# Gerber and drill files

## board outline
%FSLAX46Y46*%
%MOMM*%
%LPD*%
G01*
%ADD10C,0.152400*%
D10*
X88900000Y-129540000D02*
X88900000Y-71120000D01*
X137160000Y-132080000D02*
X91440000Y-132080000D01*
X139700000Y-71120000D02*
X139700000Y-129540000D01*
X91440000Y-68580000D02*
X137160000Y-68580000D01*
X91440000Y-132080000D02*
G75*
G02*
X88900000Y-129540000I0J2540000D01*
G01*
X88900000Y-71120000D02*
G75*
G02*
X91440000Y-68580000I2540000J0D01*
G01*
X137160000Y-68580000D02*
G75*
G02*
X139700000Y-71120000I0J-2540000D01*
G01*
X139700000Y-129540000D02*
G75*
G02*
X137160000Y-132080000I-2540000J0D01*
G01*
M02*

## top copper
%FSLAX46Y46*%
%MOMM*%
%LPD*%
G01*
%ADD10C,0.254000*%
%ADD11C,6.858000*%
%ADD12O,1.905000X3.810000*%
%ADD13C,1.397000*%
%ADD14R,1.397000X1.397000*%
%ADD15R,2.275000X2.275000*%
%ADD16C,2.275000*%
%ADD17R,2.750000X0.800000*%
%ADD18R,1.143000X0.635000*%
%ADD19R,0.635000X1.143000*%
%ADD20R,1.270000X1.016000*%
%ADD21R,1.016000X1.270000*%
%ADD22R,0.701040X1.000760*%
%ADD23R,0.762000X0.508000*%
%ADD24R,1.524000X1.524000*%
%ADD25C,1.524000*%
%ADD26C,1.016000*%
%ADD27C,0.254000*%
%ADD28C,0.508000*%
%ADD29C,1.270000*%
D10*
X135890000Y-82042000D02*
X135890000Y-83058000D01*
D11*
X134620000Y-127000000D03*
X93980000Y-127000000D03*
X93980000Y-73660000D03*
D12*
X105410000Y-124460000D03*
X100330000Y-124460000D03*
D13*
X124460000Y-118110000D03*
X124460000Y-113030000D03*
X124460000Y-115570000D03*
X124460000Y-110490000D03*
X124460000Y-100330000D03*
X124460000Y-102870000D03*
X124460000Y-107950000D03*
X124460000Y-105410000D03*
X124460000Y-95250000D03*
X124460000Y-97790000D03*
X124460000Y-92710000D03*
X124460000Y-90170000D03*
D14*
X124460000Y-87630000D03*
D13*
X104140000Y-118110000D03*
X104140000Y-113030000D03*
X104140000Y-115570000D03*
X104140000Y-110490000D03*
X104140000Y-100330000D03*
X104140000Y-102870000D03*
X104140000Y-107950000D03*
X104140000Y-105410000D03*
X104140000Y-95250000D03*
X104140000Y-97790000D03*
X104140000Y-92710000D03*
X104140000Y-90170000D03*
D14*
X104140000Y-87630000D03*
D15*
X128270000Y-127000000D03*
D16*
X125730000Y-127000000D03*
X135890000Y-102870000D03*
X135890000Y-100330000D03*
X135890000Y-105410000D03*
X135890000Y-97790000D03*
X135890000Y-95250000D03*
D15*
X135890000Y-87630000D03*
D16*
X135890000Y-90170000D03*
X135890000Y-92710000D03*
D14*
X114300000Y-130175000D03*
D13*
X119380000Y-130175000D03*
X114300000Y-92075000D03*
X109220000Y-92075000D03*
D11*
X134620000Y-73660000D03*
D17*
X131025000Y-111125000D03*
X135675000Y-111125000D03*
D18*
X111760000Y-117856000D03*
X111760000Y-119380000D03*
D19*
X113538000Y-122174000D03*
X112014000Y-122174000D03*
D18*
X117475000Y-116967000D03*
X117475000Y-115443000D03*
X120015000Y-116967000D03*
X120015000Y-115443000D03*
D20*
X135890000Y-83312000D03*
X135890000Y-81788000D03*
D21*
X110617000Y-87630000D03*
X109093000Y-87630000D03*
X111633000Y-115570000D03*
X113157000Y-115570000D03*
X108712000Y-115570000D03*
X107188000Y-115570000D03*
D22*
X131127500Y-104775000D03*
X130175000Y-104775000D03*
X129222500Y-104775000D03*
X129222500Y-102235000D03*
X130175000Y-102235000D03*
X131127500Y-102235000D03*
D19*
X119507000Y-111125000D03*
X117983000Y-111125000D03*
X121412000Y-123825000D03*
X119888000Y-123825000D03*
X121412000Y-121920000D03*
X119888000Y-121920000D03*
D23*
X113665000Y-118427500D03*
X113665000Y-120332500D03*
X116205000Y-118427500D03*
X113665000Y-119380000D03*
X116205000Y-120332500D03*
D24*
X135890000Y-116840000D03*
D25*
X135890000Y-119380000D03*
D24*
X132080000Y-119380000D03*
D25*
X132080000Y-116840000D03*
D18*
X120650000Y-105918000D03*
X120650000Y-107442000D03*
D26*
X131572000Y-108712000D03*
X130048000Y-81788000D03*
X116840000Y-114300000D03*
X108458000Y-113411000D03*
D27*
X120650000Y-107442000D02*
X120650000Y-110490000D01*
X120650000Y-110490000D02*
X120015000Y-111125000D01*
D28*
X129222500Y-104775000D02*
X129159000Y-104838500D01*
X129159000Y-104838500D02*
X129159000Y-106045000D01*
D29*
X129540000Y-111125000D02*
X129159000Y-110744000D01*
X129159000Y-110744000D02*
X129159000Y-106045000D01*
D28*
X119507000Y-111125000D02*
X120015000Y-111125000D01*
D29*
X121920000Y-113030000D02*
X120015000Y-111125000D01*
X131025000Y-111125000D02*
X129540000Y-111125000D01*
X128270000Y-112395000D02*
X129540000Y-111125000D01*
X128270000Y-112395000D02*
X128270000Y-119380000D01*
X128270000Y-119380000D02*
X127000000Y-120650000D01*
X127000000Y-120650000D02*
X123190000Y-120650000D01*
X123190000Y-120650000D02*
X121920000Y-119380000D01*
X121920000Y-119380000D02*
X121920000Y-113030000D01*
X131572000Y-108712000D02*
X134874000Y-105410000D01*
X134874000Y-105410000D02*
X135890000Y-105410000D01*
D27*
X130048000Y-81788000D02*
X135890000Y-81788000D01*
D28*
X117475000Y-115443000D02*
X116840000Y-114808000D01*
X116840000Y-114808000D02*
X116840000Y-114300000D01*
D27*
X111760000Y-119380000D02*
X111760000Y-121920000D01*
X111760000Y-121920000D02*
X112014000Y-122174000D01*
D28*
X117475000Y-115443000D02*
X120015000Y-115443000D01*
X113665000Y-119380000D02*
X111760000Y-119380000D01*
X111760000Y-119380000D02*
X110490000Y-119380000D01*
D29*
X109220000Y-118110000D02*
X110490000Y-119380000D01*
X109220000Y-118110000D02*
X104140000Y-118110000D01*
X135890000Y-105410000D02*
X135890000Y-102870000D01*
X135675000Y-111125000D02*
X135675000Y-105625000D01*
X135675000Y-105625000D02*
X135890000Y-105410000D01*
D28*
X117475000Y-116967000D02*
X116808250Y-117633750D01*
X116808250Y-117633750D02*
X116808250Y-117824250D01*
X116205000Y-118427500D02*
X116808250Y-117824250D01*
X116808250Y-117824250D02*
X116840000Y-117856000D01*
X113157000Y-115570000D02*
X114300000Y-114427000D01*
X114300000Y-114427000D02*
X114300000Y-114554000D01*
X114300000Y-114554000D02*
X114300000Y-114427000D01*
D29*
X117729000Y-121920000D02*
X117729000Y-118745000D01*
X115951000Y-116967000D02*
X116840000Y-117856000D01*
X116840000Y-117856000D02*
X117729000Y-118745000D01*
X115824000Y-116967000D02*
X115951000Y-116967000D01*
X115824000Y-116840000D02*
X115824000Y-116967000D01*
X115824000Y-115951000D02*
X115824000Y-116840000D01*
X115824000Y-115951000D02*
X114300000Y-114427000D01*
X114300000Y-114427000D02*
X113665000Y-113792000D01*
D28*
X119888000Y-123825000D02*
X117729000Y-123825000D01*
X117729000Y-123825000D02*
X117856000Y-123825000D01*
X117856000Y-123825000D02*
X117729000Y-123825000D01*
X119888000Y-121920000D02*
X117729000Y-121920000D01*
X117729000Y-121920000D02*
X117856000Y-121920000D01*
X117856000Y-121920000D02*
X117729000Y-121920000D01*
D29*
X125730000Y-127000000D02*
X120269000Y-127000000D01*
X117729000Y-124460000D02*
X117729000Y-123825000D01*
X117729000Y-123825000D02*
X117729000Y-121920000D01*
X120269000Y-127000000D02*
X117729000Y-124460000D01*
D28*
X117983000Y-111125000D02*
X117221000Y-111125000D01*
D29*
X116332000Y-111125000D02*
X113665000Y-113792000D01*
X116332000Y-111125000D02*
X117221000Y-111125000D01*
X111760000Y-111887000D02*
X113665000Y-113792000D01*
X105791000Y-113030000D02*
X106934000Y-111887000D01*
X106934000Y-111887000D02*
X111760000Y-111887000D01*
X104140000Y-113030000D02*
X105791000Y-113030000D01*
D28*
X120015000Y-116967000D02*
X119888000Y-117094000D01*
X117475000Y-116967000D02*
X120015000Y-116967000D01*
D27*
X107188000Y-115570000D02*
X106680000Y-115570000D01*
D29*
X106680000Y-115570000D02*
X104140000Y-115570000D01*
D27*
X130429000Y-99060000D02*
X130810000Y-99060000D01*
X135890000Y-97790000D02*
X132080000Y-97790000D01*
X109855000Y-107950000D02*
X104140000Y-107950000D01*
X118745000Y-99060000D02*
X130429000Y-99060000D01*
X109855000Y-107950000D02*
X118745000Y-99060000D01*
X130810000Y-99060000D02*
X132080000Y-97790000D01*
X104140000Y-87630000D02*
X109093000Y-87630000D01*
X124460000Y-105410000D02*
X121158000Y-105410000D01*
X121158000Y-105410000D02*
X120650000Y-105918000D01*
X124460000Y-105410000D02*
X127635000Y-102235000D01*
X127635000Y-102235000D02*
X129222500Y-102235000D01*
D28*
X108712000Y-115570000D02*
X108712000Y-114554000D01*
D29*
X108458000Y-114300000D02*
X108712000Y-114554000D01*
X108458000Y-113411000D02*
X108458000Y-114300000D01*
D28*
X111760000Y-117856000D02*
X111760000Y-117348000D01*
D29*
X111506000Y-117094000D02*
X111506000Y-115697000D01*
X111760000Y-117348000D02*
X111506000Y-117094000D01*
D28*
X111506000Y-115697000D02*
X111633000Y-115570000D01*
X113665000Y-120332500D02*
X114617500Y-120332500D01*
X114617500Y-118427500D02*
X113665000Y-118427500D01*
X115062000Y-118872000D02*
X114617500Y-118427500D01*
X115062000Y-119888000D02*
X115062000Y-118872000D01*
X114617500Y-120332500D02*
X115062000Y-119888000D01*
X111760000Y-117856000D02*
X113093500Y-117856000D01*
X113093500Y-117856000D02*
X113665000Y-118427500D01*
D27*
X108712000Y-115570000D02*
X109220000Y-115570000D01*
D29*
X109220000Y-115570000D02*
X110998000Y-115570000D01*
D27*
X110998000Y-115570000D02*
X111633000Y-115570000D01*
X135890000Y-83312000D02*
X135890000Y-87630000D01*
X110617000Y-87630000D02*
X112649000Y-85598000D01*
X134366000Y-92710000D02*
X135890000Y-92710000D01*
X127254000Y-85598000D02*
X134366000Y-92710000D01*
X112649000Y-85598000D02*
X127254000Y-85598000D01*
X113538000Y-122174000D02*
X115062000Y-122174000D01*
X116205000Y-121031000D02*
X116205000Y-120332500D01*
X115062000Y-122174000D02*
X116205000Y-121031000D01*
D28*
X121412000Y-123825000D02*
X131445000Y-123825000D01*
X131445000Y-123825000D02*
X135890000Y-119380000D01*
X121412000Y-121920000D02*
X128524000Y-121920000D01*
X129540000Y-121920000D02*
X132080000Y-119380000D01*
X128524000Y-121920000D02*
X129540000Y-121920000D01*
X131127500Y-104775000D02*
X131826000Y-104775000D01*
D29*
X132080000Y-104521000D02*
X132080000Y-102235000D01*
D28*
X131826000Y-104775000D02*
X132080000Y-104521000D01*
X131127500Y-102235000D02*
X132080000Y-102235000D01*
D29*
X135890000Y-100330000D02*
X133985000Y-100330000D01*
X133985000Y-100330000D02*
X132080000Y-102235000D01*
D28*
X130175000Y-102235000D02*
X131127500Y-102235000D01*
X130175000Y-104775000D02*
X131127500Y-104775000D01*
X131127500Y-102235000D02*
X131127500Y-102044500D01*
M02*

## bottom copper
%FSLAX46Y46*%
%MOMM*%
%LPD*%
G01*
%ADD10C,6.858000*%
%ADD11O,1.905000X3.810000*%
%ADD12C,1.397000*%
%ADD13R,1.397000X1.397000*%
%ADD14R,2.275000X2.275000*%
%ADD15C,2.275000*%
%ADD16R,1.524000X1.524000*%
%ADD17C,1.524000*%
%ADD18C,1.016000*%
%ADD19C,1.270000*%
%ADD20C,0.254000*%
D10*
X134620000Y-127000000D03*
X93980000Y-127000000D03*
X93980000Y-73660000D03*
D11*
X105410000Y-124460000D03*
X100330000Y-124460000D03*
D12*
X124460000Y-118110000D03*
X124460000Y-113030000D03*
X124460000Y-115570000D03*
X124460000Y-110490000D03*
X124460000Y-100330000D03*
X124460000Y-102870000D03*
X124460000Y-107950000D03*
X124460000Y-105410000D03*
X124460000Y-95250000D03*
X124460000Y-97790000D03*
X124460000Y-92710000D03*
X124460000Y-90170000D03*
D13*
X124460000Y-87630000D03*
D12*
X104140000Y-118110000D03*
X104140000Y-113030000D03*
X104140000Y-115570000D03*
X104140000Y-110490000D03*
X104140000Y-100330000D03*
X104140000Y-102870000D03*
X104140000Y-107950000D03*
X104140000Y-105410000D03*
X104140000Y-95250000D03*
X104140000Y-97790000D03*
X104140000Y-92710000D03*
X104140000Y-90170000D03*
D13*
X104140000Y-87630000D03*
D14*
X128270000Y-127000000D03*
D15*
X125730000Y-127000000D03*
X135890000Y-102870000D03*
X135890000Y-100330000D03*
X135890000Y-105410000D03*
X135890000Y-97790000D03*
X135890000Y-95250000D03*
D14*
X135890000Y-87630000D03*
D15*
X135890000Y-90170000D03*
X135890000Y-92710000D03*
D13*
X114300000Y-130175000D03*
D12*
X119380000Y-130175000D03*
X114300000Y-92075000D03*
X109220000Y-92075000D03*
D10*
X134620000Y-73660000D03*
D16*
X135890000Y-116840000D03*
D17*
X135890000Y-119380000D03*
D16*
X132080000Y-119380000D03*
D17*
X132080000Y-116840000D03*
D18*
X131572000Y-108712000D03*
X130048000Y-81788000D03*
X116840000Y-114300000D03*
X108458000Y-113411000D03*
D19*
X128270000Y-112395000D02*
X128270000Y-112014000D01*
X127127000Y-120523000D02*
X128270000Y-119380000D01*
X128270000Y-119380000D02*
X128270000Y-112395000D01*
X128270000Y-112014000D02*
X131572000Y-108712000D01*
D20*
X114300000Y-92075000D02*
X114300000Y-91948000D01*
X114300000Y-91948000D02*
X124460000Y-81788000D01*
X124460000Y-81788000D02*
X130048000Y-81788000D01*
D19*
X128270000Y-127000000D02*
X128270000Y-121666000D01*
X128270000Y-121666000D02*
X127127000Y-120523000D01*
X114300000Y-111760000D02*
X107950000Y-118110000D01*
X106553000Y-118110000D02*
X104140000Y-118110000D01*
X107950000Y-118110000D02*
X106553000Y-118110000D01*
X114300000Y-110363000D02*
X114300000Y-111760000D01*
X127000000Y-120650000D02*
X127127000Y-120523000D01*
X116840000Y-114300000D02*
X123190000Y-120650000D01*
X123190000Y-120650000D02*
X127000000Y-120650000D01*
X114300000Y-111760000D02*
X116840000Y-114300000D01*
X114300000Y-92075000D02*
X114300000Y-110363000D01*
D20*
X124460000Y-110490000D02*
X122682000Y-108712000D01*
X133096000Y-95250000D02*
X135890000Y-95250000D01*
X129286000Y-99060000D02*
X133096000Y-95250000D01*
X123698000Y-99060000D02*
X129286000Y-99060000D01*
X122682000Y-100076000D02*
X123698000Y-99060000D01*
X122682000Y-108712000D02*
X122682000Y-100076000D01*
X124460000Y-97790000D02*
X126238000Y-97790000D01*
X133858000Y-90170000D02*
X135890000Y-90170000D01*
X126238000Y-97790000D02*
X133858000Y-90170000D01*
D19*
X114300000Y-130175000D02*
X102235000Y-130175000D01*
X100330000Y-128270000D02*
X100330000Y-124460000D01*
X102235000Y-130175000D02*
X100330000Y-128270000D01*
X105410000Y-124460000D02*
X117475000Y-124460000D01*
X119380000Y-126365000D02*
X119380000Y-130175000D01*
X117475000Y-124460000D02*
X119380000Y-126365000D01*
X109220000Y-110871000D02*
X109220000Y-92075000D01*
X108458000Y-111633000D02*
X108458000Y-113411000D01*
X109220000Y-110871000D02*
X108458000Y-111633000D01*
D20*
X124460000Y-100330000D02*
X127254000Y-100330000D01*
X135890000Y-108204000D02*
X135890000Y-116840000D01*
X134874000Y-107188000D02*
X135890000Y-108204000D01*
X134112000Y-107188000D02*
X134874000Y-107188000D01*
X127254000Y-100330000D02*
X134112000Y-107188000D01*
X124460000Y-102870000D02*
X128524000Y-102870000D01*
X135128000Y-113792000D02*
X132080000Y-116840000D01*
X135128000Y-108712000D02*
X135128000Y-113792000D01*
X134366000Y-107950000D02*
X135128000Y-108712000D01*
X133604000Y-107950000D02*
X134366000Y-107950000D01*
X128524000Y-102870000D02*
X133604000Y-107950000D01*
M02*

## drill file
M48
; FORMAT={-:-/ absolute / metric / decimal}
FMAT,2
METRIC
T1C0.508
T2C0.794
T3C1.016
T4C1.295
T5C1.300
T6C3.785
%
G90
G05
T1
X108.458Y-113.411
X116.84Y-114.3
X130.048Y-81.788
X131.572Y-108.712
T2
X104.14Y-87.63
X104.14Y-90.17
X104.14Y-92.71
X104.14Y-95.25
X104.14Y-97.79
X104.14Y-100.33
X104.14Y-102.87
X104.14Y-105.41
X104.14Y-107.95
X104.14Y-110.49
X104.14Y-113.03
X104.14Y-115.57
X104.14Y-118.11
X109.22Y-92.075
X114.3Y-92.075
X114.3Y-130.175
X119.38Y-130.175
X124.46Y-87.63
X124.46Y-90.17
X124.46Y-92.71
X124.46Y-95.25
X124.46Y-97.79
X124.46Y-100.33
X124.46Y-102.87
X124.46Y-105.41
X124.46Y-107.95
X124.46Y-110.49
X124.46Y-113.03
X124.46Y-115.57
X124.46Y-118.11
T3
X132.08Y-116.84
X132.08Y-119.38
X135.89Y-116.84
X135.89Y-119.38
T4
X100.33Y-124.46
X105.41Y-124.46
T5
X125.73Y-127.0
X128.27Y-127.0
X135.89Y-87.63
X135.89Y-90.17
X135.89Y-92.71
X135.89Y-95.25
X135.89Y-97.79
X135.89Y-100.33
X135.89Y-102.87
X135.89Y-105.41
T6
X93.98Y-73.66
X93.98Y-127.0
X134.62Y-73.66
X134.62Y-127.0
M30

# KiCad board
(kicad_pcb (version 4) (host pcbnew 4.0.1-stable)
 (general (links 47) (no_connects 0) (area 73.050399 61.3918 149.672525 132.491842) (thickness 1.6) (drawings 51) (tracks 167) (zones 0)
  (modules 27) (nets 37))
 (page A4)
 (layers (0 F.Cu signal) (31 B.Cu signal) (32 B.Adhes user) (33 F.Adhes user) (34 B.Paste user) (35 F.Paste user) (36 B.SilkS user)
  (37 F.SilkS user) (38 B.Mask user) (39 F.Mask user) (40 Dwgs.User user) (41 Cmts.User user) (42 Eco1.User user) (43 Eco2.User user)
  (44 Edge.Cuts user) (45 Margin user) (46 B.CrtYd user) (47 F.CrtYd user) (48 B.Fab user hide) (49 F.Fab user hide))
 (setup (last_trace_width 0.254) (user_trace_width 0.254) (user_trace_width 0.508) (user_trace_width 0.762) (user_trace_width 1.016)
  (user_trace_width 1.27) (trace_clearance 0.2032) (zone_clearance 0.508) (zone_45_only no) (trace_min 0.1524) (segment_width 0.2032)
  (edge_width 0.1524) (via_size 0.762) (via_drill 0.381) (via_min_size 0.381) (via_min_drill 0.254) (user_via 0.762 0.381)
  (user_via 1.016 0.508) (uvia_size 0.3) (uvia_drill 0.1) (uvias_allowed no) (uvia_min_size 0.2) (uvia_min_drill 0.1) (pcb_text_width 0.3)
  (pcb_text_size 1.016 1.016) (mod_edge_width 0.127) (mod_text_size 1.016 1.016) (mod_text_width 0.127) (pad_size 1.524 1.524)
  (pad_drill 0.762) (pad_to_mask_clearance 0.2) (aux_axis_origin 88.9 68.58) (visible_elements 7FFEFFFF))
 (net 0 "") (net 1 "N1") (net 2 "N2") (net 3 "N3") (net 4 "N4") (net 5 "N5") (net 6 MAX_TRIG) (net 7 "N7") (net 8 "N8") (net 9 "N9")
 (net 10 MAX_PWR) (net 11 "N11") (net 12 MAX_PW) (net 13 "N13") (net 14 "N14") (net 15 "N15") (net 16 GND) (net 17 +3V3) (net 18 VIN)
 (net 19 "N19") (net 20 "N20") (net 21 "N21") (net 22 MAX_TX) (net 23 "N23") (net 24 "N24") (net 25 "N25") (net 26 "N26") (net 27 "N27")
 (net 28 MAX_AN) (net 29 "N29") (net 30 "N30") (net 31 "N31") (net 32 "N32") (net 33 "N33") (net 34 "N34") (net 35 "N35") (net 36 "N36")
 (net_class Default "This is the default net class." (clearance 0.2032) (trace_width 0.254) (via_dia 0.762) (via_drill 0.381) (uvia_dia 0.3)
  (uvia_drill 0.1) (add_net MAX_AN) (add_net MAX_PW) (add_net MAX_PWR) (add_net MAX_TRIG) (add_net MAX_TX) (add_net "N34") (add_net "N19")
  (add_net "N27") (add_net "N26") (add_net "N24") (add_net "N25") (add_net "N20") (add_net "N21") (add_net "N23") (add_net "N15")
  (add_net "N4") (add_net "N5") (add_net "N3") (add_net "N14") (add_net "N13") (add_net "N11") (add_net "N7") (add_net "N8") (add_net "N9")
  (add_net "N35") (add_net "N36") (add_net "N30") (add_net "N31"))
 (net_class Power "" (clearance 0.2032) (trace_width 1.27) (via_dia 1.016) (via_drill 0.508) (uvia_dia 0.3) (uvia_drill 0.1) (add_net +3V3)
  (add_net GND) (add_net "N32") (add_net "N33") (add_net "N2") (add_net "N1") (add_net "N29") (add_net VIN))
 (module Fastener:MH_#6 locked (layer F.Cu) (at 134.62 127)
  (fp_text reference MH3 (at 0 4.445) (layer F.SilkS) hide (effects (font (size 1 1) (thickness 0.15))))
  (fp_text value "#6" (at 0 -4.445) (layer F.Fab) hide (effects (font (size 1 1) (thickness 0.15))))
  (pad 1 thru_hole circle (at 0 0) (size 6.858 6.858) (drill 3.7846) (layers *.Cu *.Mask F.SilkS)))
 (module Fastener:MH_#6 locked (layer F.Cu) (at 93.98 127)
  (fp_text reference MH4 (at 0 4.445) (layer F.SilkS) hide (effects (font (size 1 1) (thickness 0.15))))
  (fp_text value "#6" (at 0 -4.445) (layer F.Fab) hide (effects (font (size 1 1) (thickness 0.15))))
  (pad 1 thru_hole circle (at 0 0) (size 6.858 6.858) (drill 3.7846) (layers *.Cu *.Mask F.SilkS)))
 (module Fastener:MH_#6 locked (layer F.Cu) (at 93.98 73.66)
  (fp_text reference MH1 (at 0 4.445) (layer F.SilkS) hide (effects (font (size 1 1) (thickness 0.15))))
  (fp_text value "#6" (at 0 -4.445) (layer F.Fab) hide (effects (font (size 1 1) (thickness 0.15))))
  (pad 1 thru_hole circle (at 0 0) (size 6.858 6.858) (drill 3.7846) (layers *.Cu *.Mask F.SilkS)))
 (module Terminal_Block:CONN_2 (layer F.Cu) (at 102.87 124.46 180)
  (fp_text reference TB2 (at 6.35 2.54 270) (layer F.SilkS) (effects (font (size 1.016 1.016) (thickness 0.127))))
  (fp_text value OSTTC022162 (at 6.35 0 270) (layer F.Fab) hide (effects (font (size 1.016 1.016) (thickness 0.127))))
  (pad 1 thru_hole oval (at -2.54 0 180) (size 1.905 3.81) (drill 1.2954) (layers *.Cu F.Paste F.SilkS F.Mask) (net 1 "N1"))
  (pad 2 thru_hole oval (at 2.54 0 180) (size 1.905 3.81) (drill 1.2954) (layers *.Cu F.Paste F.SilkS F.Mask) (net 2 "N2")))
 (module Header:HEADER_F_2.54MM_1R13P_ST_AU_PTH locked (layer F.Cu) (at 124.46 102.87 270)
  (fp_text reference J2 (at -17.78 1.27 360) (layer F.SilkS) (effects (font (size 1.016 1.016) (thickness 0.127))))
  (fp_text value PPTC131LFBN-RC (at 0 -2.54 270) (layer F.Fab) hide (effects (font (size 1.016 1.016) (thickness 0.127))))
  (pad 13 thru_hole circle (at 15.24 0 270) (size 1.397 1.397) (drill 0.79375) (layers *.Cu *.Mask F.SilkS) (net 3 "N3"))
  (pad 11 thru_hole circle (at 10.16 0 270) (size 1.397 1.397) (drill 0.79375) (layers *.Cu *.Mask F.SilkS) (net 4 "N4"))
  (pad 12 thru_hole circle (at 12.7 0 270) (size 1.397 1.397) (drill 0.79375) (layers *.Cu *.Mask F.SilkS) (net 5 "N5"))
  (pad 10 thru_hole circle (at 7.62 0 270) (size 1.397 1.397) (drill 0.79375) (layers *.Cu *.Mask F.SilkS) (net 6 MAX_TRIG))
  (pad 6 thru_hole circle (at -2.54 0 270) (size 1.397 1.397) (drill 0.79375) (layers *.Cu *.Mask F.SilkS) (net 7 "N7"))
  (pad 7 thru_hole circle (at 0 0 270) (size 1.397 1.397) (drill 0.79375) (layers *.Cu *.Mask F.SilkS) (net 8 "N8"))
  (pad 9 thru_hole circle (at 5.08 0 270) (size 1.397 1.397) (drill 0.79375) (layers *.Cu *.Mask F.SilkS) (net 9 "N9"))
  (pad 8 thru_hole circle (at 2.54 0 270) (size 1.397 1.397) (drill 0.79375) (layers *.Cu *.Mask F.SilkS) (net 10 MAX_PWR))
  (pad 4 thru_hole circle (at -7.62 0 270) (size 1.397 1.397) (drill 0.79375) (layers *.Cu *.Mask F.SilkS) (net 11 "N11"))
  (pad 5 thru_hole circle (at -5.08 0 270) (size 1.397 1.397) (drill 0.79375) (layers *.Cu *.Mask F.SilkS) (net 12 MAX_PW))
  (pad 3 thru_hole circle (at -10.16 0 270) (size 1.397 1.397) (drill 0.79375) (layers *.Cu *.Mask F.SilkS) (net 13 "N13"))
  (pad 2 thru_hole circle (at -12.7 0 270) (size 1.397 1.397) (drill 0.79375) (layers *.Cu *.Mask F.SilkS) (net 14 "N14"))
  (pad 1 thru_hole rect (at -15.24 0 270) (size 1.397 1.397) (drill 0.79375) (layers *.Cu *.Mask F.SilkS) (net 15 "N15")))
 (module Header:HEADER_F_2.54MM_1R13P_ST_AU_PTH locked (layer F.Cu) (at 104.14 102.87 270)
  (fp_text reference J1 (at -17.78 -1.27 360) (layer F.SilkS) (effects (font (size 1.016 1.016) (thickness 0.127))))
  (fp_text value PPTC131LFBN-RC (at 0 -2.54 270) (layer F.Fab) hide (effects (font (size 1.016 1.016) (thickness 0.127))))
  (pad 13 thru_hole circle (at 15.24 0 270) (size 1.397 1.397) (drill 0.79375) (layers *.Cu *.Mask F.SilkS) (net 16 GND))
  (pad 11 thru_hole circle (at 10.16 0 270) (size 1.397 1.397) (drill 0.79375) (layers *.Cu *.Mask F.SilkS) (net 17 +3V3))
  (pad 12 thru_hole circle (at 12.7 0 270) (size 1.397 1.397) (drill 0.79375) (layers *.Cu *.Mask F.SilkS) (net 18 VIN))
  (pad 10 thru_hole circle (at 7.62 0 270) (size 1.397 1.397) (drill 0.79375) (layers *.Cu *.Mask F.SilkS) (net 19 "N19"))
  (pad 6 thru_hole circle (at -2.54 0 270) (size 1.397 1.397) (drill 0.79375) (layers *.Cu *.Mask F.SilkS) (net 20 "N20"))
  (pad 7 thru_hole circle (at 0 0 270) (size 1.397 1.397) (drill 0.79375) (layers *.Cu *.Mask F.SilkS) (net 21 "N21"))
  (pad 9 thru_hole circle (at 5.08 0 270) (size 1.397 1.397) (drill 0.79375) (layers *.Cu *.Mask F.SilkS) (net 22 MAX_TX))
  (pad 8 thru_hole circle (at 2.54 0 270) (size 1.397 1.397) (drill 0.79375) (layers *.Cu *.Mask F.SilkS) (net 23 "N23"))
  (pad 4 thru_hole circle (at -7.62 0 270) (size 1.397 1.397) (drill 0.79375) (layers *.Cu *.Mask F.SilkS) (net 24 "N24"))
  (pad 5 thru_hole circle (at -5.08 0 270) (size 1.397 1.397) (drill 0.79375) (layers *.Cu *.Mask F.SilkS) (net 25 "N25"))
  (pad 3 thru_hole circle (at -10.16 0 270) (size 1.397 1.397) (drill 0.79375) (layers *.Cu *.Mask F.SilkS) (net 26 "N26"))
  (pad 2 thru_hole circle (at -12.7 0 270) (size 1.397 1.397) (drill 0.79375) (layers *.Cu *.Mask F.SilkS) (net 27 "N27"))
  (pad 1 thru_hole rect (at -15.24 0 270) (size 1.397 1.397) (drill 0.79375) (layers *.Cu *.Mask F.SilkS) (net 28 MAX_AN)))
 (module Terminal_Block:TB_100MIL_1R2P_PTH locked (layer F.Cu) (at 127 127 180)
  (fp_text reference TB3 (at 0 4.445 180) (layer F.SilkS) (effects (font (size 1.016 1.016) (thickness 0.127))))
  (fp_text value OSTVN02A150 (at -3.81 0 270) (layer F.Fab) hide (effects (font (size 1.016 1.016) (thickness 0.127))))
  (pad 1 thru_hole rect (at -1.27 0 180) (size 2.275 2.275) (drill 1.3) (layers *.Cu *.Mask F.SilkS) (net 16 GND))
  (pad 2 thru_hole circle (at 1.27 0 180) (size 2.275 2.275) (drill 1.3) (layers *.Cu *.Mask F.SilkS) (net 17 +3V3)))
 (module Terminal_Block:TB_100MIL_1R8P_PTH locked (layer F.Cu) (at 135.89 96.52 270)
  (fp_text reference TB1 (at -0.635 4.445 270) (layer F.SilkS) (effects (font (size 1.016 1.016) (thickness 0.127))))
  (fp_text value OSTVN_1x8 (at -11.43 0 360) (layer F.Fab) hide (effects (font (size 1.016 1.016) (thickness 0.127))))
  (pad 7 thru_hole circle (at 6.35 0 270) (size 2.275 2.275) (drill 1.3) (layers *.Cu *.Mask F.SilkS) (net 16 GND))
  (pad 6 thru_hole circle (at 3.81 0 270) (size 2.275 2.275) (drill 1.3) (layers *.Cu *.Mask F.SilkS) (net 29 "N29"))
  (pad 8 thru_hole circle (at 8.89 0 270) (size 2.275 2.275) (drill 1.3) (layers *.Cu *.Mask F.SilkS) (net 16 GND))
  (pad 5 thru_hole circle (at 1.27 0 270) (size 2.275 2.275) (drill 1.3) (layers *.Cu *.Mask F.SilkS) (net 22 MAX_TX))
  (pad 4 thru_hole circle (at -1.27 0 270) (size 2.275 2.275) (drill 1.3) (layers *.Cu *.Mask F.SilkS) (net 6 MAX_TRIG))
  (pad 1 thru_hole rect (at -8.89 0 270) (size 2.275 2.275) (drill 1.3) (layers *.Cu *.Mask F.SilkS) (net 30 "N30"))
  (pad 2 thru_hole circle (at -6.35 0 270) (size 2.275 2.275) (drill 1.3) (layers *.Cu *.Mask F.SilkS) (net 12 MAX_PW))
  (pad 3 thru_hole circle (at -3.81 0 270) (size 2.275 2.275) (drill 1.3) (layers *.Cu *.Mask F.SilkS) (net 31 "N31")))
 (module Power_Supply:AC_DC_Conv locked (layer B.Cu) (at 114.3 111.125 90)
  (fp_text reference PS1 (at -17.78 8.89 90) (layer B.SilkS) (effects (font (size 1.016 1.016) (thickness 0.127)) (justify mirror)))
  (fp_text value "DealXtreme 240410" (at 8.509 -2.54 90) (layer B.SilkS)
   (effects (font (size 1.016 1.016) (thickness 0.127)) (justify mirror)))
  (pad 1 thru_hole rect (at -19.05 0 90) (size 1.397 1.397) (drill 0.79375) (layers *.Cu *.Mask B.SilkS) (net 2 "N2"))
  (pad 2 thru_hole circle (at -19.05 5.08 90) (size 1.397 1.397) (drill 0.79375) (layers *.Cu *.Mask B.SilkS) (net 1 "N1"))
  (pad 4 thru_hole circle (at 19.05 0 90) (size 1.397 1.397) (drill 0.79375) (layers *.Cu *.Mask B.SilkS) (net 16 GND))
  (pad 3 thru_hole circle (at 19.05 -5.08 90) (size 1.397 1.397) (drill 0.79375) (layers *.Cu *.Mask B.SilkS) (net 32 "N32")))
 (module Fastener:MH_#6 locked (layer F.Cu) (at 134.62 73.66)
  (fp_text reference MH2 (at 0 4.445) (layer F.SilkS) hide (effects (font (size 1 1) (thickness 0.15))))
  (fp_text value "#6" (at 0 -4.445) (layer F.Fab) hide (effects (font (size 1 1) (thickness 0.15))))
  (pad 1 thru_hole circle (at 0 0) (size 6.858 6.858) (drill 3.7846) (layers *.Cu *.Mask F.SilkS)))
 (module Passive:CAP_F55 (layer F.Cu) (at 133.35 111.125 90)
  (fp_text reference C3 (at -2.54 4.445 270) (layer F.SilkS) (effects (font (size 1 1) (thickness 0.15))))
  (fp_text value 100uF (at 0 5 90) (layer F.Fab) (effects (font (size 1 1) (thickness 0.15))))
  (pad 1 smd rect (at 0 -2.325 90) (size 0.8 2.75) (layers F.Cu F.Paste F.Mask) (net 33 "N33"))
  (pad 2 smd rect (at 0 2.325 90) (size 0.8 2.75) (layers F.Cu F.Paste F.Mask) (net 16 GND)))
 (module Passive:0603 (layer F.Cu) (at 111.76 118.618 270)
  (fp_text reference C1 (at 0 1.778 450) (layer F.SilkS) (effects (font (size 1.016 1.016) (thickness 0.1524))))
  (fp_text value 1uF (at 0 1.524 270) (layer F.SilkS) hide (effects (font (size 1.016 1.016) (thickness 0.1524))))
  (pad 1 smd rect (at -0.762 0 270) (size 0.635 1.143) (layers F.Cu F.Paste F.Mask) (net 32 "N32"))
  (pad 2 smd rect (at 0.762 0 270) (size 0.635 1.143) (layers F.Cu F.Paste F.Mask) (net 16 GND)))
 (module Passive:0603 (layer F.Cu) (at 112.776 122.174 180)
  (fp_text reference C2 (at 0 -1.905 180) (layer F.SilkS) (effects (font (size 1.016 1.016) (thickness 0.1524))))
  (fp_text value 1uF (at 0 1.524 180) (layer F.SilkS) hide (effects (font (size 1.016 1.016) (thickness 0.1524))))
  (pad 1 smd rect (at -0.762 0 180) (size 0.635 1.143) (layers F.Cu F.Paste F.Mask) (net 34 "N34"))
  (pad 2 smd rect (at 0.762 0 180) (size 0.635 1.143) (layers F.Cu F.Paste F.Mask) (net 16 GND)))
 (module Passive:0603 (layer F.Cu) (at 117.475 116.205 90)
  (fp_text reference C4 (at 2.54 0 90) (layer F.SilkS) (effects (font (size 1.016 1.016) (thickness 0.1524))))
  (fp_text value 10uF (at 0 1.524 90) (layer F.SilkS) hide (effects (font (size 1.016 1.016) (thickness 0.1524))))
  (pad 1 smd rect (at -0.762 0 90) (size 0.635 1.143) (layers F.Cu F.Paste F.Mask) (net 17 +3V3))
  (pad 2 smd rect (at 0.762 0 90) (size 0.635 1.143) (layers F.Cu F.Paste F.Mask) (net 16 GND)))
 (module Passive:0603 (layer F.Cu) (at 120.015 116.205 90)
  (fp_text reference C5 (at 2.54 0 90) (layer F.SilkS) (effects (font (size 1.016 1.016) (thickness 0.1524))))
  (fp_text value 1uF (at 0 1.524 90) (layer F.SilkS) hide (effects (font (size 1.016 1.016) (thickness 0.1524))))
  (pad 1 smd rect (at -0.762 0 90) (size 0.635 1.143) (layers F.Cu F.Paste F.Mask) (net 17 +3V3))
  (pad 2 smd rect (at 0.762 0 90) (size 0.635 1.143) (layers F.Cu F.Paste F.Mask) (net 16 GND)))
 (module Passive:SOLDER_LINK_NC (layer F.Cu) (at 135.89 82.55 180)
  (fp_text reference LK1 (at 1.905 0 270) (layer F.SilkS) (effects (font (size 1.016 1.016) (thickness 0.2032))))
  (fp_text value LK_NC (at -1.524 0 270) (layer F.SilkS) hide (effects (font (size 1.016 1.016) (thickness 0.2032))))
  (fp_line (start 0 0.508) (end 0 -0.508) (layer F.Cu) (width 0.254))
  (pad 1 smd rect (at 0 -0.762 180) (size 1.27 1.016) (layers F.Cu F.Mask) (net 30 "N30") (solder_mask_margin 0.254))
  (pad 2 smd rect (at 0 0.762 180) (size 1.27 1.016) (layers F.Cu F.Mask) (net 16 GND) (solder_mask_margin 0.254)))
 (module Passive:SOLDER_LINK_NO (layer F.Cu) (at 109.855 87.63 270)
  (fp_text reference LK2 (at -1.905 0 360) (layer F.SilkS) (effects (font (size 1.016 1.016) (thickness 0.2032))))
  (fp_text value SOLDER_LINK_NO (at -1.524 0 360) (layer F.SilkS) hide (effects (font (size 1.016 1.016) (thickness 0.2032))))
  (pad 1 smd rect (at 0 -0.762 270) (size 1.27 1.016) (layers F.Cu F.Mask) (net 31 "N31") (solder_mask_margin 0.254))
  (pad 2 smd rect (at 0 0.762 270) (size 1.27 1.016) (layers F.Cu F.Mask) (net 28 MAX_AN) (solder_mask_margin 0.254)))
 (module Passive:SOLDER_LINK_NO (layer F.Cu) (at 112.395 115.57 90)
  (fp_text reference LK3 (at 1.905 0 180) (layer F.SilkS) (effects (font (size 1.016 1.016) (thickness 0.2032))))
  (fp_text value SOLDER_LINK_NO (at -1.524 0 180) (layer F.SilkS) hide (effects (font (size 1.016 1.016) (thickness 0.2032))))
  (pad 1 smd rect (at 0 -0.762 90) (size 1.27 1.016) (layers F.Cu F.Mask) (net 32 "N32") (solder_mask_margin 0.254))
  (pad 2 smd rect (at 0 0.762 90) (size 1.27 1.016) (layers F.Cu F.Mask) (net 17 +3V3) (solder_mask_margin 0.254)))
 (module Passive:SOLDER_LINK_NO (layer F.Cu) (at 107.95 115.57 270)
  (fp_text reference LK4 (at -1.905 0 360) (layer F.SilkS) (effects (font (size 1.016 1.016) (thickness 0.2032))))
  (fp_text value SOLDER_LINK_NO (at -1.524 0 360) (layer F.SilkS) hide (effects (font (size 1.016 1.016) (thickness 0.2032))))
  (pad 1 smd rect (at 0 -0.762 270) (size 1.27 1.016) (layers F.Cu F.Mask) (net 32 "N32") (solder_mask_margin 0.254))
  (pad 2 smd rect (at 0 0.762 270) (size 1.27 1.016) (layers F.Cu F.Mask) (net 18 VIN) (solder_mask_margin 0.254)))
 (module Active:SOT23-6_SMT (layer F.Cu) (at 130.175 103.505 270)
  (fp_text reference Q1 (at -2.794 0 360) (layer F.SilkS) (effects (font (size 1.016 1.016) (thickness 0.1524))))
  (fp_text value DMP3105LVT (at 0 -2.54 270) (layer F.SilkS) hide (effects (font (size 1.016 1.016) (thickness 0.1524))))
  (pad 6 smd rect (at 1.27 -0.9525 180) (size 0.70104 1.00076) (layers F.Cu F.Paste F.Mask) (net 29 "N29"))
  (pad 5 smd rect (at 1.27 0 180) (size 0.70104 1.00076) (layers F.Cu F.Paste F.Mask) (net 29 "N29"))
  (pad 4 smd rect (at 1.27 0.9525 180) (size 0.70104 1.00076) (layers F.Cu F.Paste F.Mask) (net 33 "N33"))
  (pad 3 smd rect (at -1.27 0.9525 180) (size 0.70104 1.00076) (layers F.Cu F.Paste F.Mask) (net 10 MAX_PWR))
  (pad 2 smd rect (at -1.27 0 180) (size 0.70104 1.00076) (layers F.Cu F.Paste F.Mask) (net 29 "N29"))
  (pad 1 smd rect (at -1.27 -0.9525 180) (size 0.70104 1.00076) (layers F.Cu F.Paste F.Mask) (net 29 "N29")))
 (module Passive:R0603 (layer F.Cu) (at 118.745 111.125 180)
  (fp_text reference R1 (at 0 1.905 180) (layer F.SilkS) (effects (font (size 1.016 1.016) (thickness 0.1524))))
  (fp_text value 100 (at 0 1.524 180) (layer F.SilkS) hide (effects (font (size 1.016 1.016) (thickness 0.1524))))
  (pad 1 smd rect (at -0.762 0 180) (size 0.635 1.143) (layers F.Cu F.Paste F.Mask) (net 33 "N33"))
  (pad 2 smd rect (at 0.762 0 180) (size 0.635 1.143) (layers F.Cu F.Paste F.Mask) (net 17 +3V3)))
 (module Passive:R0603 (layer F.Cu) (at 120.65 123.825 180)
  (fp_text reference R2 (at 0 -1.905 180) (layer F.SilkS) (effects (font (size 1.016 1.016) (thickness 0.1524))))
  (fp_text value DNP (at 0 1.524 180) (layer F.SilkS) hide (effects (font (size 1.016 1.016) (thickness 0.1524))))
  (pad 1 smd rect (at -0.762 0 180) (size 0.635 1.143) (layers F.Cu F.Paste F.Mask) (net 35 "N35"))
  (pad 2 smd rect (at 0.762 0 180) (size 0.635 1.143) (layers F.Cu F.Paste F.Mask) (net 17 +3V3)))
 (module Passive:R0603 (layer F.Cu) (at 120.65 121.92 180)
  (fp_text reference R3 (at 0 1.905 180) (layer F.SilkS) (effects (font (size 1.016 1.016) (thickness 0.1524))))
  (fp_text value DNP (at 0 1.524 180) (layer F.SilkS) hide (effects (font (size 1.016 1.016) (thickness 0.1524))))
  (pad 1 smd rect (at -0.762 0 180) (size 0.635 1.143) (layers F.Cu F.Paste F.Mask) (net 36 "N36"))
  (pad 2 smd rect (at 0.762 0 180) (size 0.635 1.143) (layers F.Cu F.Paste F.Mask) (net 17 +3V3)))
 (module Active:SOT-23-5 (layer F.Cu) (at 114.935 119.38)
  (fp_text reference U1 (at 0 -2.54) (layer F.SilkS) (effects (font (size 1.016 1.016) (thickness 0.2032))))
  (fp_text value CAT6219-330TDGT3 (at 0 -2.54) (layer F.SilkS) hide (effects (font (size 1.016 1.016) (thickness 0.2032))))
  (pad 1 smd rect (at -1.27 -0.9525 270) (size 0.508 0.762) (layers F.Cu F.Paste F.Mask) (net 32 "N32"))
  (pad 3 smd rect (at -1.27 0.9525 270) (size 0.508 0.762) (layers F.Cu F.Paste F.Mask) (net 32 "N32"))
  (pad 5 smd rect (at 1.27 -0.9525 270) (size 0.508 0.762) (layers F.Cu F.Paste F.Mask) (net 17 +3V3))
  (pad 2 smd rect (at -1.27 0 270) (size 0.508 0.762) (layers F.Cu F.Paste F.Mask) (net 16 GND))
  (pad 4 smd rect (at 1.27 0.9525 270) (size 0.508 0.762) (layers F.Cu F.Paste F.Mask) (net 34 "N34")))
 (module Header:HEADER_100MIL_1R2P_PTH (layer F.Cu) (at 135.89 118.11 270)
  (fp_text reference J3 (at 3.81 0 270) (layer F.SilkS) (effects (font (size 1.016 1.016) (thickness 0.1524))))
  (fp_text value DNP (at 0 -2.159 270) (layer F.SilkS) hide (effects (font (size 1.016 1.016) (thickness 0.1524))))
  (pad 1 thru_hole rect (at -1.27 0 270) (size 1.524 1.524) (drill 1.016) (layers *.Cu *.Mask F.SilkS) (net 7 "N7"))
  (pad 2 thru_hole circle (at 1.27 0 270) (size 1.524 1.524) (drill 1.016) (layers *.Cu *.Mask F.SilkS) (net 35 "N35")))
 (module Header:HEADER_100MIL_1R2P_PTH (layer F.Cu) (at 132.08 118.11 90)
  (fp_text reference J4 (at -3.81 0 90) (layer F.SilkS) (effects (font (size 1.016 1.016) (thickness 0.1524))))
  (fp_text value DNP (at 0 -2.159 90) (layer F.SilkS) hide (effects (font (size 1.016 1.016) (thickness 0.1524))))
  (pad 1 thru_hole rect (at -1.27 0 90) (size 1.524 1.524) (drill 1.016) (layers *.Cu *.Mask F.SilkS) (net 36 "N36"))
  (pad 2 thru_hole circle (at 1.27 0 90) (size 1.524 1.524) (drill 1.016) (layers *.Cu *.Mask F.SilkS) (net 8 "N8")))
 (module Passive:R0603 (layer F.Cu) (at 120.65 106.68 270)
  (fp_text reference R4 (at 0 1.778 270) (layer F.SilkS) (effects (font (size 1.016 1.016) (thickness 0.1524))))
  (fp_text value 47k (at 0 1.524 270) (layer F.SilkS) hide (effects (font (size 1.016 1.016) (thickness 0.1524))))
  (pad 1 smd rect (at -0.762 0 270) (size 0.635 1.143) (layers F.Cu F.Paste F.Mask) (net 10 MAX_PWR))
  (pad 2 smd rect (at 0.762 0 270) (size 0.635 1.143) (layers F.Cu F.Paste F.Mask) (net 33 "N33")))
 (gr_line (start 88.9 129.54) (end 88.9 71.12) (angle 90) (layer Edge.Cuts) (width 0.1524))
 (gr_line (start 137.16 132.08) (end 91.44 132.08) (angle 90) (layer Edge.Cuts) (width 0.1524))
 (gr_line (start 139.7 71.12) (end 139.7 129.54) (angle 90) (layer Edge.Cuts) (width 0.1524))
 (gr_line (start 91.44 68.58) (end 137.16 68.58) (angle 90) (layer Edge.Cuts) (width 0.1524))
 (gr_arc (start 91.44 129.54) (end 91.44 132.08) (angle 90) (layer Edge.Cuts) (width 0.1524))
 (gr_arc (start 91.44 71.12) (end 88.9 71.12) (angle 90) (layer Edge.Cuts) (width 0.1524))
 (gr_arc (start 137.16 71.12) (end 137.16 68.58) (angle 90) (layer Edge.Cuts) (width 0.1524))
 (gr_arc (start 137.16 129.54) (end 139.7 129.54) (angle 90) (layer Edge.Cuts) (width 0.1524))
 (segment (start 120.65 107.442) (end 120.65 110.49) (width 0.254) (layer F.Cu) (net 33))
 (segment (start 120.65 110.49) (end 120.015 111.125) (width 0.254) (layer F.Cu) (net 33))
 (segment (start 129.2225 104.775) (end 129.159 104.8385) (width 0.508) (layer F.Cu) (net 33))
 (segment (start 129.159 104.8385) (end 129.159 106.045) (width 0.508) (layer F.Cu) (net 33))
 (segment (start 129.54 111.125) (end 129.159 110.744) (width 1.27) (layer F.Cu) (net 33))
 (segment (start 129.159 110.744) (end 129.159 106.045) (width 1.27) (layer F.Cu) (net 33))
 (segment (start 119.507 111.125) (end 120.015 111.125) (width 0.508) (layer F.Cu) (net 33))
 (segment (start 121.92 113.03) (end 120.015 111.125) (width 1.27) (layer F.Cu) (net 33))
 (segment (start 131.025 111.125) (end 129.54 111.125) (width 1.27) (layer F.Cu) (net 33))
 (segment (start 128.27 112.395) (end 129.54 111.125) (width 1.27) (layer F.Cu) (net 33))
 (segment (start 128.27 112.395) (end 128.27 119.38) (width 1.27) (layer F.Cu) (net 33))
 (segment (start 128.27 119.38) (end 127 120.65) (width 1.27) (layer F.Cu) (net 33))
 (segment (start 127 120.65) (end 123.19 120.65) (width 1.27) (layer F.Cu) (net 33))
 (segment (start 123.19 120.65) (end 121.92 119.38) (width 1.27) (layer F.Cu) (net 33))
 (segment (start 121.92 119.38) (end 121.92 113.03) (width 1.27) (layer F.Cu) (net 33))
 (segment (start 128.27 112.395) (end 128.27 112.014) (width 1.27) (layer B.Cu) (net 16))
 (segment (start 127.127 120.523) (end 128.27 119.38) (width 1.27) (layer B.Cu) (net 16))
 (segment (start 128.27 119.38) (end 128.27 112.395) (width 1.27) (layer B.Cu) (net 16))
 (segment (start 131.572 108.712) (end 134.874 105.41) (width 1.27) (layer F.Cu) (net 16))
 (via (at 131.572 108.712) (size 1.016) (drill 0.508) (layers F.Cu B.Cu) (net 16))
 (segment (start 128.27 112.014) (end 131.572 108.712) (width 1.27) (layer B.Cu) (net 16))
 (segment (start 134.874 105.41) (end 135.89 105.41) (width 1.27) (layer F.Cu) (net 16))
 (segment (start 114.3 92.075) (end 114.3 91.948) (width 0.254) (layer B.Cu) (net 16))
 (segment (start 114.3 91.948) (end 124.46 81.788) (width 0.254) (layer B.Cu) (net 16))
 (segment (start 130.048 81.788) (end 135.89 81.788) (width 0.254) (layer F.Cu) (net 16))
 (via (at 130.048 81.788) (size 1.016) (drill 0.508) (layers F.Cu B.Cu) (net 16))
 (segment (start 124.46 81.788) (end 130.048 81.788) (width 0.254) (layer B.Cu) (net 16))
 (segment (start 117.475 115.443) (end 116.84 114.808) (width 0.508) (layer F.Cu) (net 16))
 (via (at 116.84 114.3) (size 1.016) (drill 0.508) (layers F.Cu B.Cu) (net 16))
 (segment (start 116.84 114.808) (end 116.84 114.3) (width 0.508) (layer F.Cu) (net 16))
 (segment (start 128.27 127) (end 128.27 121.666) (width 1.27) (layer B.Cu) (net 16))
 (segment (start 128.27 121.666) (end 127.127 120.523) (width 1.27) (layer B.Cu) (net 16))
 (segment (start 114.3 111.76) (end 107.95 118.11) (width 1.27) (layer B.Cu) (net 16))
 (segment (start 106.553 118.11) (end 104.14 118.11) (width 1.27) (layer B.Cu) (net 16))
 (segment (start 107.95 118.11) (end 106.553 118.11) (width 1.27) (layer B.Cu) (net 16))
 (segment (start 114.3 110.363) (end 114.3 111.76) (width 1.27) (layer B.Cu) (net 16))
 (segment (start 127 120.65) (end 127.127 120.523) (width 1.27) (layer B.Cu) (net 16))
 (segment (start 116.84 114.3) (end 123.19 120.65) (width 1.27) (layer B.Cu) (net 16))
 (segment (start 123.19 120.65) (end 127 120.65) (width 1.27) (layer B.Cu) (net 16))
 (segment (start 114.3 111.76) (end 116.84 114.3) (width 1.27) (layer B.Cu) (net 16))
 (segment (start 114.3 92.075) (end 114.3 110.363) (width 1.27) (layer B.Cu) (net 16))
 (segment (start 111.76 119.38) (end 111.76 121.92) (width 0.254) (layer F.Cu) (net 16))
 (segment (start 111.76 121.92) (end 112.014 122.174) (width 0.254) (layer F.Cu) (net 16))
 (segment (start 117.475 115.443) (end 120.015 115.443) (width 0.508) (layer F.Cu) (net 16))
 (segment (start 113.665 119.38) (end 111.76 119.38) (width 0.508) (layer F.Cu) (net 16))
 (segment (start 111.76 119.38) (end 110.49 119.38) (width 0.508) (layer F.Cu) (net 16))
 (segment (start 109.22 118.11) (end 110.49 119.38) (width 1.27) (layer F.Cu) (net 16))
 (segment (start 109.22 118.11) (end 104.14 118.11) (width 1.27) (layer F.Cu) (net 16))
 (segment (start 135.89 105.41) (end 135.89 102.87) (width 1.27) (layer F.Cu) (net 16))
 (segment (start 135.675 111.125) (end 135.675 105.625) (width 1.27) (layer F.Cu) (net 16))
 (segment (start 135.675 105.625) (end 135.89 105.41) (width 1.27) (layer F.Cu) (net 16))
 (segment (start 117.475 116.967) (end 116.80825 117.63375) (width 0.508) (layer F.Cu) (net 17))
 (segment (start 116.80825 117.63375) (end 116.80825 117.82425) (width 0.508) (layer F.Cu) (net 17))
 (segment (start 116.205 118.4275) (end 116.80825 117.82425) (width 0.508) (layer F.Cu) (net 17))
 (segment (start 116.80825 117.82425) (end 116.84 117.856) (width 0.508) (layer F.Cu) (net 17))
 (segment (start 113.157 115.57) (end 114.3 114.427) (width 0.508) (layer F.Cu) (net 17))
 (segment (start 114.3 114.427) (end 114.3 114.554) (width 0.508) (layer F.Cu) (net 17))
 (segment (start 114.3 114.554) (end 114.3 114.427) (width 0.508) (layer F.Cu) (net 17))
 (segment (start 117.729 121.92) (end 117.729 118.745) (width 1.27) (layer F.Cu) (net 17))
 (segment (start 115.951 116.967) (end 116.84 117.856) (width 1.27) (layer F.Cu) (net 17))
 (segment (start 116.84 117.856) (end 117.729 118.745) (width 1.27) (layer F.Cu) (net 17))
 (segment (start 115.824 116.967) (end 115.951 116.967) (width 1.27) (layer F.Cu) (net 17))
 (segment (start 115.824 116.84) (end 115.824 116.967) (width 1.27) (layer F.Cu) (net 17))
 (segment (start 115.824 115.951) (end 115.824 116.84) (width 1.27) (layer F.Cu) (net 17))
 (segment (start 115.824 115.951) (end 114.3 114.427) (width 1.27) (layer F.Cu) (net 17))
 (segment (start 114.3 114.427) (end 113.665 113.792) (width 1.27) (layer F.Cu) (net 17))
 (segment (start 119.888 123.825) (end 117.729 123.825) (width 0.508) (layer F.Cu) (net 17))
 (segment (start 117.729 123.825) (end 117.856 123.825) (width 0.508) (layer F.Cu) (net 17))
 (segment (start 117.856 123.825) (end 117.729 123.825) (width 0.508) (layer F.Cu) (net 17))
 (segment (start 119.888 121.92) (end 117.729 121.92) (width 0.508) (layer F.Cu) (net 17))
 (segment (start 117.729 121.92) (end 117.856 121.92) (width 0.508) (layer F.Cu) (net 17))
 (segment (start 117.856 121.92) (end 117.729 121.92) (width 0.508) (layer F.Cu) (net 17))
 (segment (start 125.73 127) (end 120.269 127) (width 1.27) (layer F.Cu) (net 17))
 (segment (start 117.729 124.46) (end 117.729 123.825) (width 1.27) (layer F.Cu) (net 17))
 (segment (start 117.729 123.825) (end 117.729 121.92) (width 1.27) (layer F.Cu) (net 17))
 (segment (start 120.269 127) (end 117.729 124.46) (width 1.27) (layer F.Cu) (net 17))
 (segment (start 117.983 111.125) (end 117.221 111.125) (width 0.508) (layer F.Cu) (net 17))
 (segment (start 116.332 111.125) (end 113.665 113.792) (width 1.27) (layer F.Cu) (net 17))
 (segment (start 116.332 111.125) (end 117.221 111.125) (width 1.27) (layer F.Cu) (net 17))
 (segment (start 111.76 111.887) (end 113.665 113.792) (width 1.27) (layer F.Cu) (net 17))
 (segment (start 105.791 113.03) (end 106.934 111.887) (width 1.27) (layer F.Cu) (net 17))
 (segment (start 106.934 111.887) (end 111.76 111.887) (width 1.27) (layer F.Cu) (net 17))
 (segment (start 104.14 113.03) (end 105.791 113.03) (width 1.27) (layer F.Cu) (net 17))
 (segment (start 120.015 116.967) (end 119.888 117.094) (width 0.508) (layer F.Cu) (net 17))
 (segment (start 117.475 116.967) (end 120.015 116.967) (width 0.508) (layer F.Cu) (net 17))
 (segment (start 107.188 115.57) (end 106.68 115.57) (width 0.254) (layer F.Cu) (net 18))
 (segment (start 106.68 115.57) (end 104.14 115.57) (width 1.27) (layer F.Cu) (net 18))
 (segment (start 130.429 99.06) (end 130.81 99.06) (width 0.254) (layer F.Cu) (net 22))
 (segment (start 135.89 97.79) (end 132.08 97.79) (width 0.254) (layer F.Cu) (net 22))
 (segment (start 109.855 107.95) (end 104.14 107.95) (width 0.254) (layer F.Cu) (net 22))
 (segment (start 118.745 99.06) (end 130.429 99.06) (width 0.254) (layer F.Cu) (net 22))
 (segment (start 109.855 107.95) (end 118.745 99.06) (width 0.254) (layer F.Cu) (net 22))
 (segment (start 130.81 99.06) (end 132.08 97.79) (width 0.254) (layer F.Cu) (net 22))
 (segment (start 104.14 87.63) (end 109.093 87.63) (width 0.254) (layer F.Cu) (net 28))
 (segment (start 124.46 110.49) (end 122.682 108.712) (width 0.254) (layer B.Cu) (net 6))
 (segment (start 133.096 95.25) (end 135.89 95.25) (width 0.254) (layer B.Cu) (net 6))
 (segment (start 129.286 99.06) (end 133.096 95.25) (width 0.254) (layer B.Cu) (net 6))
 (segment (start 123.698 99.06) (end 129.286 99.06) (width 0.254) (layer B.Cu) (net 6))
 (segment (start 122.682 100.076) (end 123.698 99.06) (width 0.254) (layer B.Cu) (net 6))
 (segment (start 122.682 108.712) (end 122.682 100.076) (width 0.254) (layer B.Cu) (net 6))
 (segment (start 124.46 105.41) (end 121.158 105.41) (width 0.254) (layer F.Cu) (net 10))
 (segment (start 121.158 105.41) (end 120.65 105.918) (width 0.254) (layer F.Cu) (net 10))
 (segment (start 124.46 105.41) (end 127.635 102.235) (width 0.254) (layer F.Cu) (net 10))
 (segment (start 127.635 102.235) (end 129.2225 102.235) (width 0.254) (layer F.Cu) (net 10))
 (segment (start 124.46 97.79) (end 126.238 97.79) (width 0.254) (layer B.Cu) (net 12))
 (segment (start 133.858 90.17) (end 135.89 90.17) (width 0.254) (layer B.Cu) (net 12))
 (segment (start 126.238 97.79) (end 133.858 90.17) (width 0.254) (layer B.Cu) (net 12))
 (segment (start 114.3 130.175) (end 102.235 130.175) (width 1.27) (layer B.Cu) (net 2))
 (segment (start 100.33 128.27) (end 100.33 124.46) (width 1.27) (layer B.Cu) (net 2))
 (segment (start 102.235 130.175) (end 100.33 128.27) (width 1.27) (layer B.Cu) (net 2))
 (segment (start 105.41 124.46) (end 117.475 124.46) (width 1.27) (layer B.Cu) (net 1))
 (segment (start 119.38 126.365) (end 119.38 130.175) (width 1.27) (layer B.Cu) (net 1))
 (segment (start 117.475 124.46) (end 119.38 126.365) (width 1.27) (layer B.Cu) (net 1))
 (segment (start 108.712 115.57) (end 108.712 114.554) (width 0.508) (layer F.Cu) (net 32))
 (segment (start 108.458 114.3) (end 108.712 114.554) (width 1.27) (layer F.Cu) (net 32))
 (segment (start 109.22 110.871) (end 109.22 92.075) (width 1.27) (layer B.Cu) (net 32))
 (via (at 108.458 113.411) (size 1.016) (drill 0.508) (layers F.Cu B.Cu) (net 32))
 (segment (start 108.458 111.633) (end 108.458 113.411) (width 1.27) (layer B.Cu) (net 32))
 (segment (start 109.22 110.871) (end 108.458 111.633) (width 1.27) (layer B.Cu) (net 32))
 (segment (start 108.458 113.411) (end 108.458 114.3) (width 1.27) (layer F.Cu) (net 32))
 (segment (start 111.76 117.856) (end 111.76 117.348) (width 0.508) (layer F.Cu) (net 32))
 (segment (start 111.506 117.094) (end 111.506 115.697) (width 1.27) (layer F.Cu) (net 32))
 (segment (start 111.76 117.348) (end 111.506 117.094) (width 1.27) (layer F.Cu) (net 32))
 (segment (start 111.506 115.697) (end 111.633 115.57) (width 0.508) (layer F.Cu) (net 32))
 (segment (start 113.665 120.3325) (end 114.6175 120.3325) (width 0.508) (layer F.Cu) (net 32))
 (segment (start 114.6175 118.4275) (end 113.665 118.4275) (width 0.508) (layer F.Cu) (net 32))
 (segment (start 115.062 118.872) (end 114.6175 118.4275) (width 0.508) (layer F.Cu) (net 32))
 (segment (start 115.062 119.888) (end 115.062 118.872) (width 0.508) (layer F.Cu) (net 32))
 (segment (start 114.6175 120.3325) (end 115.062 119.888) (width 0.508) (layer F.Cu) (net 32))
 (segment (start 111.76 117.856) (end 113.0935 117.856) (width 0.508) (layer F.Cu) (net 32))
 (segment (start 113.0935 117.856) (end 113.665 118.4275) (width 0.508) (layer F.Cu) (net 32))
 (segment (start 108.712 115.57) (end 109.22 115.57) (width 0.254) (layer F.Cu) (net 32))
 (segment (start 109.22 115.57) (end 110.998 115.57) (width 1.27) (layer F.Cu) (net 32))
 (segment (start 110.998 115.57) (end 111.633 115.57) (width 0.254) (layer F.Cu) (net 32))
 (segment (start 135.89 83.312) (end 135.89 87.63) (width 0.254) (layer F.Cu) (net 30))
 (segment (start 110.617 87.63) (end 112.649 85.598) (width 0.254) (layer F.Cu) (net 31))
 (segment (start 134.366 92.71) (end 135.89 92.71) (width 0.254) (layer F.Cu) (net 31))
 (segment (start 127.254 85.598) (end 134.366 92.71) (width 0.254) (layer F.Cu) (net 31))
 (segment (start 112.649 85.598) (end 127.254 85.598) (width 0.254) (layer F.Cu) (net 31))
 (segment (start 113.538 122.174) (end 115.062 122.174) (width 0.254) (layer F.Cu) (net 34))
 (segment (start 116.205 121.031) (end 116.205 120.3325) (width 0.254) (layer F.Cu) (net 34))
 (segment (start 115.062 122.174) (end 116.205 121.031) (width 0.254) (layer F.Cu) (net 34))
 (segment (start 124.46 100.33) (end 127.254 100.33) (width 0.254) (layer B.Cu) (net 7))
 (segment (start 135.89 108.204) (end 135.89 116.84) (width 0.254) (layer B.Cu) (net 7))
 (segment (start 134.874 107.188) (end 135.89 108.204) (width 0.254) (layer B.Cu) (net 7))
 (segment (start 134.112 107.188) (end 134.874 107.188) (width 0.254) (layer B.Cu) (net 7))
 (segment (start 127.254 100.33) (end 134.112 107.188) (width 0.254) (layer B.Cu) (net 7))
 (segment (start 124.46 102.87) (end 128.524 102.87) (width 0.254) (layer B.Cu) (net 8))
 (segment (start 135.128 113.792) (end 132.08 116.84) (width 0.254) (layer B.Cu) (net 8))
 (segment (start 135.128 108.712) (end 135.128 113.792) (width 0.254) (layer B.Cu) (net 8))
 (segment (start 134.366 107.95) (end 135.128 108.712) (width 0.254) (layer B.Cu) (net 8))
 (segment (start 133.604 107.95) (end 134.366 107.95) (width 0.254) (layer B.Cu) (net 8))
 (segment (start 128.524 102.87) (end 133.604 107.95) (width 0.254) (layer B.Cu) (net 8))
 (segment (start 121.412 123.825) (end 131.445 123.825) (width 0.508) (layer F.Cu) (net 35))
 (segment (start 131.445 123.825) (end 135.89 119.38) (width 0.508) (layer F.Cu) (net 35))
 (segment (start 121.412 121.92) (end 128.524 121.92) (width 0.508) (layer F.Cu) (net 36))
 (segment (start 129.54 121.92) (end 132.08 119.38) (width 0.508) (layer F.Cu) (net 36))
 (segment (start 128.524 121.92) (end 129.54 121.92) (width 0.508) (layer F.Cu) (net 36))
 (segment (start 131.1275 104.775) (end 131.826 104.775) (width 0.508) (layer F.Cu) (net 29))
 (segment (start 132.08 104.521) (end 132.08 102.235) (width 1.27) (layer F.Cu) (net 29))
 (segment (start 131.826 104.775) (end 132.08 104.521) (width 0.508) (layer F.Cu) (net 29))
 (segment (start 131.1275 102.235) (end 132.08 102.235) (width 0.508) (layer F.Cu) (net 29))
 (segment (start 135.89 100.33) (end 133.985 100.33) (width 1.27) (layer F.Cu) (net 29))
 (segment (start 133.985 100.33) (end 132.08 102.235) (width 1.27) (layer F.Cu) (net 29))
 (segment (start 130.175 102.235) (end 131.1275 102.235) (width 0.508) (layer F.Cu) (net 29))
 (segment (start 130.175 104.775) (end 131.1275 104.775) (width 0.508) (layer F.Cu) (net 29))
 (segment (start 131.1275 102.235) (end 131.1275 102.0445) (width 0.508) (layer F.Cu) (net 29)))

